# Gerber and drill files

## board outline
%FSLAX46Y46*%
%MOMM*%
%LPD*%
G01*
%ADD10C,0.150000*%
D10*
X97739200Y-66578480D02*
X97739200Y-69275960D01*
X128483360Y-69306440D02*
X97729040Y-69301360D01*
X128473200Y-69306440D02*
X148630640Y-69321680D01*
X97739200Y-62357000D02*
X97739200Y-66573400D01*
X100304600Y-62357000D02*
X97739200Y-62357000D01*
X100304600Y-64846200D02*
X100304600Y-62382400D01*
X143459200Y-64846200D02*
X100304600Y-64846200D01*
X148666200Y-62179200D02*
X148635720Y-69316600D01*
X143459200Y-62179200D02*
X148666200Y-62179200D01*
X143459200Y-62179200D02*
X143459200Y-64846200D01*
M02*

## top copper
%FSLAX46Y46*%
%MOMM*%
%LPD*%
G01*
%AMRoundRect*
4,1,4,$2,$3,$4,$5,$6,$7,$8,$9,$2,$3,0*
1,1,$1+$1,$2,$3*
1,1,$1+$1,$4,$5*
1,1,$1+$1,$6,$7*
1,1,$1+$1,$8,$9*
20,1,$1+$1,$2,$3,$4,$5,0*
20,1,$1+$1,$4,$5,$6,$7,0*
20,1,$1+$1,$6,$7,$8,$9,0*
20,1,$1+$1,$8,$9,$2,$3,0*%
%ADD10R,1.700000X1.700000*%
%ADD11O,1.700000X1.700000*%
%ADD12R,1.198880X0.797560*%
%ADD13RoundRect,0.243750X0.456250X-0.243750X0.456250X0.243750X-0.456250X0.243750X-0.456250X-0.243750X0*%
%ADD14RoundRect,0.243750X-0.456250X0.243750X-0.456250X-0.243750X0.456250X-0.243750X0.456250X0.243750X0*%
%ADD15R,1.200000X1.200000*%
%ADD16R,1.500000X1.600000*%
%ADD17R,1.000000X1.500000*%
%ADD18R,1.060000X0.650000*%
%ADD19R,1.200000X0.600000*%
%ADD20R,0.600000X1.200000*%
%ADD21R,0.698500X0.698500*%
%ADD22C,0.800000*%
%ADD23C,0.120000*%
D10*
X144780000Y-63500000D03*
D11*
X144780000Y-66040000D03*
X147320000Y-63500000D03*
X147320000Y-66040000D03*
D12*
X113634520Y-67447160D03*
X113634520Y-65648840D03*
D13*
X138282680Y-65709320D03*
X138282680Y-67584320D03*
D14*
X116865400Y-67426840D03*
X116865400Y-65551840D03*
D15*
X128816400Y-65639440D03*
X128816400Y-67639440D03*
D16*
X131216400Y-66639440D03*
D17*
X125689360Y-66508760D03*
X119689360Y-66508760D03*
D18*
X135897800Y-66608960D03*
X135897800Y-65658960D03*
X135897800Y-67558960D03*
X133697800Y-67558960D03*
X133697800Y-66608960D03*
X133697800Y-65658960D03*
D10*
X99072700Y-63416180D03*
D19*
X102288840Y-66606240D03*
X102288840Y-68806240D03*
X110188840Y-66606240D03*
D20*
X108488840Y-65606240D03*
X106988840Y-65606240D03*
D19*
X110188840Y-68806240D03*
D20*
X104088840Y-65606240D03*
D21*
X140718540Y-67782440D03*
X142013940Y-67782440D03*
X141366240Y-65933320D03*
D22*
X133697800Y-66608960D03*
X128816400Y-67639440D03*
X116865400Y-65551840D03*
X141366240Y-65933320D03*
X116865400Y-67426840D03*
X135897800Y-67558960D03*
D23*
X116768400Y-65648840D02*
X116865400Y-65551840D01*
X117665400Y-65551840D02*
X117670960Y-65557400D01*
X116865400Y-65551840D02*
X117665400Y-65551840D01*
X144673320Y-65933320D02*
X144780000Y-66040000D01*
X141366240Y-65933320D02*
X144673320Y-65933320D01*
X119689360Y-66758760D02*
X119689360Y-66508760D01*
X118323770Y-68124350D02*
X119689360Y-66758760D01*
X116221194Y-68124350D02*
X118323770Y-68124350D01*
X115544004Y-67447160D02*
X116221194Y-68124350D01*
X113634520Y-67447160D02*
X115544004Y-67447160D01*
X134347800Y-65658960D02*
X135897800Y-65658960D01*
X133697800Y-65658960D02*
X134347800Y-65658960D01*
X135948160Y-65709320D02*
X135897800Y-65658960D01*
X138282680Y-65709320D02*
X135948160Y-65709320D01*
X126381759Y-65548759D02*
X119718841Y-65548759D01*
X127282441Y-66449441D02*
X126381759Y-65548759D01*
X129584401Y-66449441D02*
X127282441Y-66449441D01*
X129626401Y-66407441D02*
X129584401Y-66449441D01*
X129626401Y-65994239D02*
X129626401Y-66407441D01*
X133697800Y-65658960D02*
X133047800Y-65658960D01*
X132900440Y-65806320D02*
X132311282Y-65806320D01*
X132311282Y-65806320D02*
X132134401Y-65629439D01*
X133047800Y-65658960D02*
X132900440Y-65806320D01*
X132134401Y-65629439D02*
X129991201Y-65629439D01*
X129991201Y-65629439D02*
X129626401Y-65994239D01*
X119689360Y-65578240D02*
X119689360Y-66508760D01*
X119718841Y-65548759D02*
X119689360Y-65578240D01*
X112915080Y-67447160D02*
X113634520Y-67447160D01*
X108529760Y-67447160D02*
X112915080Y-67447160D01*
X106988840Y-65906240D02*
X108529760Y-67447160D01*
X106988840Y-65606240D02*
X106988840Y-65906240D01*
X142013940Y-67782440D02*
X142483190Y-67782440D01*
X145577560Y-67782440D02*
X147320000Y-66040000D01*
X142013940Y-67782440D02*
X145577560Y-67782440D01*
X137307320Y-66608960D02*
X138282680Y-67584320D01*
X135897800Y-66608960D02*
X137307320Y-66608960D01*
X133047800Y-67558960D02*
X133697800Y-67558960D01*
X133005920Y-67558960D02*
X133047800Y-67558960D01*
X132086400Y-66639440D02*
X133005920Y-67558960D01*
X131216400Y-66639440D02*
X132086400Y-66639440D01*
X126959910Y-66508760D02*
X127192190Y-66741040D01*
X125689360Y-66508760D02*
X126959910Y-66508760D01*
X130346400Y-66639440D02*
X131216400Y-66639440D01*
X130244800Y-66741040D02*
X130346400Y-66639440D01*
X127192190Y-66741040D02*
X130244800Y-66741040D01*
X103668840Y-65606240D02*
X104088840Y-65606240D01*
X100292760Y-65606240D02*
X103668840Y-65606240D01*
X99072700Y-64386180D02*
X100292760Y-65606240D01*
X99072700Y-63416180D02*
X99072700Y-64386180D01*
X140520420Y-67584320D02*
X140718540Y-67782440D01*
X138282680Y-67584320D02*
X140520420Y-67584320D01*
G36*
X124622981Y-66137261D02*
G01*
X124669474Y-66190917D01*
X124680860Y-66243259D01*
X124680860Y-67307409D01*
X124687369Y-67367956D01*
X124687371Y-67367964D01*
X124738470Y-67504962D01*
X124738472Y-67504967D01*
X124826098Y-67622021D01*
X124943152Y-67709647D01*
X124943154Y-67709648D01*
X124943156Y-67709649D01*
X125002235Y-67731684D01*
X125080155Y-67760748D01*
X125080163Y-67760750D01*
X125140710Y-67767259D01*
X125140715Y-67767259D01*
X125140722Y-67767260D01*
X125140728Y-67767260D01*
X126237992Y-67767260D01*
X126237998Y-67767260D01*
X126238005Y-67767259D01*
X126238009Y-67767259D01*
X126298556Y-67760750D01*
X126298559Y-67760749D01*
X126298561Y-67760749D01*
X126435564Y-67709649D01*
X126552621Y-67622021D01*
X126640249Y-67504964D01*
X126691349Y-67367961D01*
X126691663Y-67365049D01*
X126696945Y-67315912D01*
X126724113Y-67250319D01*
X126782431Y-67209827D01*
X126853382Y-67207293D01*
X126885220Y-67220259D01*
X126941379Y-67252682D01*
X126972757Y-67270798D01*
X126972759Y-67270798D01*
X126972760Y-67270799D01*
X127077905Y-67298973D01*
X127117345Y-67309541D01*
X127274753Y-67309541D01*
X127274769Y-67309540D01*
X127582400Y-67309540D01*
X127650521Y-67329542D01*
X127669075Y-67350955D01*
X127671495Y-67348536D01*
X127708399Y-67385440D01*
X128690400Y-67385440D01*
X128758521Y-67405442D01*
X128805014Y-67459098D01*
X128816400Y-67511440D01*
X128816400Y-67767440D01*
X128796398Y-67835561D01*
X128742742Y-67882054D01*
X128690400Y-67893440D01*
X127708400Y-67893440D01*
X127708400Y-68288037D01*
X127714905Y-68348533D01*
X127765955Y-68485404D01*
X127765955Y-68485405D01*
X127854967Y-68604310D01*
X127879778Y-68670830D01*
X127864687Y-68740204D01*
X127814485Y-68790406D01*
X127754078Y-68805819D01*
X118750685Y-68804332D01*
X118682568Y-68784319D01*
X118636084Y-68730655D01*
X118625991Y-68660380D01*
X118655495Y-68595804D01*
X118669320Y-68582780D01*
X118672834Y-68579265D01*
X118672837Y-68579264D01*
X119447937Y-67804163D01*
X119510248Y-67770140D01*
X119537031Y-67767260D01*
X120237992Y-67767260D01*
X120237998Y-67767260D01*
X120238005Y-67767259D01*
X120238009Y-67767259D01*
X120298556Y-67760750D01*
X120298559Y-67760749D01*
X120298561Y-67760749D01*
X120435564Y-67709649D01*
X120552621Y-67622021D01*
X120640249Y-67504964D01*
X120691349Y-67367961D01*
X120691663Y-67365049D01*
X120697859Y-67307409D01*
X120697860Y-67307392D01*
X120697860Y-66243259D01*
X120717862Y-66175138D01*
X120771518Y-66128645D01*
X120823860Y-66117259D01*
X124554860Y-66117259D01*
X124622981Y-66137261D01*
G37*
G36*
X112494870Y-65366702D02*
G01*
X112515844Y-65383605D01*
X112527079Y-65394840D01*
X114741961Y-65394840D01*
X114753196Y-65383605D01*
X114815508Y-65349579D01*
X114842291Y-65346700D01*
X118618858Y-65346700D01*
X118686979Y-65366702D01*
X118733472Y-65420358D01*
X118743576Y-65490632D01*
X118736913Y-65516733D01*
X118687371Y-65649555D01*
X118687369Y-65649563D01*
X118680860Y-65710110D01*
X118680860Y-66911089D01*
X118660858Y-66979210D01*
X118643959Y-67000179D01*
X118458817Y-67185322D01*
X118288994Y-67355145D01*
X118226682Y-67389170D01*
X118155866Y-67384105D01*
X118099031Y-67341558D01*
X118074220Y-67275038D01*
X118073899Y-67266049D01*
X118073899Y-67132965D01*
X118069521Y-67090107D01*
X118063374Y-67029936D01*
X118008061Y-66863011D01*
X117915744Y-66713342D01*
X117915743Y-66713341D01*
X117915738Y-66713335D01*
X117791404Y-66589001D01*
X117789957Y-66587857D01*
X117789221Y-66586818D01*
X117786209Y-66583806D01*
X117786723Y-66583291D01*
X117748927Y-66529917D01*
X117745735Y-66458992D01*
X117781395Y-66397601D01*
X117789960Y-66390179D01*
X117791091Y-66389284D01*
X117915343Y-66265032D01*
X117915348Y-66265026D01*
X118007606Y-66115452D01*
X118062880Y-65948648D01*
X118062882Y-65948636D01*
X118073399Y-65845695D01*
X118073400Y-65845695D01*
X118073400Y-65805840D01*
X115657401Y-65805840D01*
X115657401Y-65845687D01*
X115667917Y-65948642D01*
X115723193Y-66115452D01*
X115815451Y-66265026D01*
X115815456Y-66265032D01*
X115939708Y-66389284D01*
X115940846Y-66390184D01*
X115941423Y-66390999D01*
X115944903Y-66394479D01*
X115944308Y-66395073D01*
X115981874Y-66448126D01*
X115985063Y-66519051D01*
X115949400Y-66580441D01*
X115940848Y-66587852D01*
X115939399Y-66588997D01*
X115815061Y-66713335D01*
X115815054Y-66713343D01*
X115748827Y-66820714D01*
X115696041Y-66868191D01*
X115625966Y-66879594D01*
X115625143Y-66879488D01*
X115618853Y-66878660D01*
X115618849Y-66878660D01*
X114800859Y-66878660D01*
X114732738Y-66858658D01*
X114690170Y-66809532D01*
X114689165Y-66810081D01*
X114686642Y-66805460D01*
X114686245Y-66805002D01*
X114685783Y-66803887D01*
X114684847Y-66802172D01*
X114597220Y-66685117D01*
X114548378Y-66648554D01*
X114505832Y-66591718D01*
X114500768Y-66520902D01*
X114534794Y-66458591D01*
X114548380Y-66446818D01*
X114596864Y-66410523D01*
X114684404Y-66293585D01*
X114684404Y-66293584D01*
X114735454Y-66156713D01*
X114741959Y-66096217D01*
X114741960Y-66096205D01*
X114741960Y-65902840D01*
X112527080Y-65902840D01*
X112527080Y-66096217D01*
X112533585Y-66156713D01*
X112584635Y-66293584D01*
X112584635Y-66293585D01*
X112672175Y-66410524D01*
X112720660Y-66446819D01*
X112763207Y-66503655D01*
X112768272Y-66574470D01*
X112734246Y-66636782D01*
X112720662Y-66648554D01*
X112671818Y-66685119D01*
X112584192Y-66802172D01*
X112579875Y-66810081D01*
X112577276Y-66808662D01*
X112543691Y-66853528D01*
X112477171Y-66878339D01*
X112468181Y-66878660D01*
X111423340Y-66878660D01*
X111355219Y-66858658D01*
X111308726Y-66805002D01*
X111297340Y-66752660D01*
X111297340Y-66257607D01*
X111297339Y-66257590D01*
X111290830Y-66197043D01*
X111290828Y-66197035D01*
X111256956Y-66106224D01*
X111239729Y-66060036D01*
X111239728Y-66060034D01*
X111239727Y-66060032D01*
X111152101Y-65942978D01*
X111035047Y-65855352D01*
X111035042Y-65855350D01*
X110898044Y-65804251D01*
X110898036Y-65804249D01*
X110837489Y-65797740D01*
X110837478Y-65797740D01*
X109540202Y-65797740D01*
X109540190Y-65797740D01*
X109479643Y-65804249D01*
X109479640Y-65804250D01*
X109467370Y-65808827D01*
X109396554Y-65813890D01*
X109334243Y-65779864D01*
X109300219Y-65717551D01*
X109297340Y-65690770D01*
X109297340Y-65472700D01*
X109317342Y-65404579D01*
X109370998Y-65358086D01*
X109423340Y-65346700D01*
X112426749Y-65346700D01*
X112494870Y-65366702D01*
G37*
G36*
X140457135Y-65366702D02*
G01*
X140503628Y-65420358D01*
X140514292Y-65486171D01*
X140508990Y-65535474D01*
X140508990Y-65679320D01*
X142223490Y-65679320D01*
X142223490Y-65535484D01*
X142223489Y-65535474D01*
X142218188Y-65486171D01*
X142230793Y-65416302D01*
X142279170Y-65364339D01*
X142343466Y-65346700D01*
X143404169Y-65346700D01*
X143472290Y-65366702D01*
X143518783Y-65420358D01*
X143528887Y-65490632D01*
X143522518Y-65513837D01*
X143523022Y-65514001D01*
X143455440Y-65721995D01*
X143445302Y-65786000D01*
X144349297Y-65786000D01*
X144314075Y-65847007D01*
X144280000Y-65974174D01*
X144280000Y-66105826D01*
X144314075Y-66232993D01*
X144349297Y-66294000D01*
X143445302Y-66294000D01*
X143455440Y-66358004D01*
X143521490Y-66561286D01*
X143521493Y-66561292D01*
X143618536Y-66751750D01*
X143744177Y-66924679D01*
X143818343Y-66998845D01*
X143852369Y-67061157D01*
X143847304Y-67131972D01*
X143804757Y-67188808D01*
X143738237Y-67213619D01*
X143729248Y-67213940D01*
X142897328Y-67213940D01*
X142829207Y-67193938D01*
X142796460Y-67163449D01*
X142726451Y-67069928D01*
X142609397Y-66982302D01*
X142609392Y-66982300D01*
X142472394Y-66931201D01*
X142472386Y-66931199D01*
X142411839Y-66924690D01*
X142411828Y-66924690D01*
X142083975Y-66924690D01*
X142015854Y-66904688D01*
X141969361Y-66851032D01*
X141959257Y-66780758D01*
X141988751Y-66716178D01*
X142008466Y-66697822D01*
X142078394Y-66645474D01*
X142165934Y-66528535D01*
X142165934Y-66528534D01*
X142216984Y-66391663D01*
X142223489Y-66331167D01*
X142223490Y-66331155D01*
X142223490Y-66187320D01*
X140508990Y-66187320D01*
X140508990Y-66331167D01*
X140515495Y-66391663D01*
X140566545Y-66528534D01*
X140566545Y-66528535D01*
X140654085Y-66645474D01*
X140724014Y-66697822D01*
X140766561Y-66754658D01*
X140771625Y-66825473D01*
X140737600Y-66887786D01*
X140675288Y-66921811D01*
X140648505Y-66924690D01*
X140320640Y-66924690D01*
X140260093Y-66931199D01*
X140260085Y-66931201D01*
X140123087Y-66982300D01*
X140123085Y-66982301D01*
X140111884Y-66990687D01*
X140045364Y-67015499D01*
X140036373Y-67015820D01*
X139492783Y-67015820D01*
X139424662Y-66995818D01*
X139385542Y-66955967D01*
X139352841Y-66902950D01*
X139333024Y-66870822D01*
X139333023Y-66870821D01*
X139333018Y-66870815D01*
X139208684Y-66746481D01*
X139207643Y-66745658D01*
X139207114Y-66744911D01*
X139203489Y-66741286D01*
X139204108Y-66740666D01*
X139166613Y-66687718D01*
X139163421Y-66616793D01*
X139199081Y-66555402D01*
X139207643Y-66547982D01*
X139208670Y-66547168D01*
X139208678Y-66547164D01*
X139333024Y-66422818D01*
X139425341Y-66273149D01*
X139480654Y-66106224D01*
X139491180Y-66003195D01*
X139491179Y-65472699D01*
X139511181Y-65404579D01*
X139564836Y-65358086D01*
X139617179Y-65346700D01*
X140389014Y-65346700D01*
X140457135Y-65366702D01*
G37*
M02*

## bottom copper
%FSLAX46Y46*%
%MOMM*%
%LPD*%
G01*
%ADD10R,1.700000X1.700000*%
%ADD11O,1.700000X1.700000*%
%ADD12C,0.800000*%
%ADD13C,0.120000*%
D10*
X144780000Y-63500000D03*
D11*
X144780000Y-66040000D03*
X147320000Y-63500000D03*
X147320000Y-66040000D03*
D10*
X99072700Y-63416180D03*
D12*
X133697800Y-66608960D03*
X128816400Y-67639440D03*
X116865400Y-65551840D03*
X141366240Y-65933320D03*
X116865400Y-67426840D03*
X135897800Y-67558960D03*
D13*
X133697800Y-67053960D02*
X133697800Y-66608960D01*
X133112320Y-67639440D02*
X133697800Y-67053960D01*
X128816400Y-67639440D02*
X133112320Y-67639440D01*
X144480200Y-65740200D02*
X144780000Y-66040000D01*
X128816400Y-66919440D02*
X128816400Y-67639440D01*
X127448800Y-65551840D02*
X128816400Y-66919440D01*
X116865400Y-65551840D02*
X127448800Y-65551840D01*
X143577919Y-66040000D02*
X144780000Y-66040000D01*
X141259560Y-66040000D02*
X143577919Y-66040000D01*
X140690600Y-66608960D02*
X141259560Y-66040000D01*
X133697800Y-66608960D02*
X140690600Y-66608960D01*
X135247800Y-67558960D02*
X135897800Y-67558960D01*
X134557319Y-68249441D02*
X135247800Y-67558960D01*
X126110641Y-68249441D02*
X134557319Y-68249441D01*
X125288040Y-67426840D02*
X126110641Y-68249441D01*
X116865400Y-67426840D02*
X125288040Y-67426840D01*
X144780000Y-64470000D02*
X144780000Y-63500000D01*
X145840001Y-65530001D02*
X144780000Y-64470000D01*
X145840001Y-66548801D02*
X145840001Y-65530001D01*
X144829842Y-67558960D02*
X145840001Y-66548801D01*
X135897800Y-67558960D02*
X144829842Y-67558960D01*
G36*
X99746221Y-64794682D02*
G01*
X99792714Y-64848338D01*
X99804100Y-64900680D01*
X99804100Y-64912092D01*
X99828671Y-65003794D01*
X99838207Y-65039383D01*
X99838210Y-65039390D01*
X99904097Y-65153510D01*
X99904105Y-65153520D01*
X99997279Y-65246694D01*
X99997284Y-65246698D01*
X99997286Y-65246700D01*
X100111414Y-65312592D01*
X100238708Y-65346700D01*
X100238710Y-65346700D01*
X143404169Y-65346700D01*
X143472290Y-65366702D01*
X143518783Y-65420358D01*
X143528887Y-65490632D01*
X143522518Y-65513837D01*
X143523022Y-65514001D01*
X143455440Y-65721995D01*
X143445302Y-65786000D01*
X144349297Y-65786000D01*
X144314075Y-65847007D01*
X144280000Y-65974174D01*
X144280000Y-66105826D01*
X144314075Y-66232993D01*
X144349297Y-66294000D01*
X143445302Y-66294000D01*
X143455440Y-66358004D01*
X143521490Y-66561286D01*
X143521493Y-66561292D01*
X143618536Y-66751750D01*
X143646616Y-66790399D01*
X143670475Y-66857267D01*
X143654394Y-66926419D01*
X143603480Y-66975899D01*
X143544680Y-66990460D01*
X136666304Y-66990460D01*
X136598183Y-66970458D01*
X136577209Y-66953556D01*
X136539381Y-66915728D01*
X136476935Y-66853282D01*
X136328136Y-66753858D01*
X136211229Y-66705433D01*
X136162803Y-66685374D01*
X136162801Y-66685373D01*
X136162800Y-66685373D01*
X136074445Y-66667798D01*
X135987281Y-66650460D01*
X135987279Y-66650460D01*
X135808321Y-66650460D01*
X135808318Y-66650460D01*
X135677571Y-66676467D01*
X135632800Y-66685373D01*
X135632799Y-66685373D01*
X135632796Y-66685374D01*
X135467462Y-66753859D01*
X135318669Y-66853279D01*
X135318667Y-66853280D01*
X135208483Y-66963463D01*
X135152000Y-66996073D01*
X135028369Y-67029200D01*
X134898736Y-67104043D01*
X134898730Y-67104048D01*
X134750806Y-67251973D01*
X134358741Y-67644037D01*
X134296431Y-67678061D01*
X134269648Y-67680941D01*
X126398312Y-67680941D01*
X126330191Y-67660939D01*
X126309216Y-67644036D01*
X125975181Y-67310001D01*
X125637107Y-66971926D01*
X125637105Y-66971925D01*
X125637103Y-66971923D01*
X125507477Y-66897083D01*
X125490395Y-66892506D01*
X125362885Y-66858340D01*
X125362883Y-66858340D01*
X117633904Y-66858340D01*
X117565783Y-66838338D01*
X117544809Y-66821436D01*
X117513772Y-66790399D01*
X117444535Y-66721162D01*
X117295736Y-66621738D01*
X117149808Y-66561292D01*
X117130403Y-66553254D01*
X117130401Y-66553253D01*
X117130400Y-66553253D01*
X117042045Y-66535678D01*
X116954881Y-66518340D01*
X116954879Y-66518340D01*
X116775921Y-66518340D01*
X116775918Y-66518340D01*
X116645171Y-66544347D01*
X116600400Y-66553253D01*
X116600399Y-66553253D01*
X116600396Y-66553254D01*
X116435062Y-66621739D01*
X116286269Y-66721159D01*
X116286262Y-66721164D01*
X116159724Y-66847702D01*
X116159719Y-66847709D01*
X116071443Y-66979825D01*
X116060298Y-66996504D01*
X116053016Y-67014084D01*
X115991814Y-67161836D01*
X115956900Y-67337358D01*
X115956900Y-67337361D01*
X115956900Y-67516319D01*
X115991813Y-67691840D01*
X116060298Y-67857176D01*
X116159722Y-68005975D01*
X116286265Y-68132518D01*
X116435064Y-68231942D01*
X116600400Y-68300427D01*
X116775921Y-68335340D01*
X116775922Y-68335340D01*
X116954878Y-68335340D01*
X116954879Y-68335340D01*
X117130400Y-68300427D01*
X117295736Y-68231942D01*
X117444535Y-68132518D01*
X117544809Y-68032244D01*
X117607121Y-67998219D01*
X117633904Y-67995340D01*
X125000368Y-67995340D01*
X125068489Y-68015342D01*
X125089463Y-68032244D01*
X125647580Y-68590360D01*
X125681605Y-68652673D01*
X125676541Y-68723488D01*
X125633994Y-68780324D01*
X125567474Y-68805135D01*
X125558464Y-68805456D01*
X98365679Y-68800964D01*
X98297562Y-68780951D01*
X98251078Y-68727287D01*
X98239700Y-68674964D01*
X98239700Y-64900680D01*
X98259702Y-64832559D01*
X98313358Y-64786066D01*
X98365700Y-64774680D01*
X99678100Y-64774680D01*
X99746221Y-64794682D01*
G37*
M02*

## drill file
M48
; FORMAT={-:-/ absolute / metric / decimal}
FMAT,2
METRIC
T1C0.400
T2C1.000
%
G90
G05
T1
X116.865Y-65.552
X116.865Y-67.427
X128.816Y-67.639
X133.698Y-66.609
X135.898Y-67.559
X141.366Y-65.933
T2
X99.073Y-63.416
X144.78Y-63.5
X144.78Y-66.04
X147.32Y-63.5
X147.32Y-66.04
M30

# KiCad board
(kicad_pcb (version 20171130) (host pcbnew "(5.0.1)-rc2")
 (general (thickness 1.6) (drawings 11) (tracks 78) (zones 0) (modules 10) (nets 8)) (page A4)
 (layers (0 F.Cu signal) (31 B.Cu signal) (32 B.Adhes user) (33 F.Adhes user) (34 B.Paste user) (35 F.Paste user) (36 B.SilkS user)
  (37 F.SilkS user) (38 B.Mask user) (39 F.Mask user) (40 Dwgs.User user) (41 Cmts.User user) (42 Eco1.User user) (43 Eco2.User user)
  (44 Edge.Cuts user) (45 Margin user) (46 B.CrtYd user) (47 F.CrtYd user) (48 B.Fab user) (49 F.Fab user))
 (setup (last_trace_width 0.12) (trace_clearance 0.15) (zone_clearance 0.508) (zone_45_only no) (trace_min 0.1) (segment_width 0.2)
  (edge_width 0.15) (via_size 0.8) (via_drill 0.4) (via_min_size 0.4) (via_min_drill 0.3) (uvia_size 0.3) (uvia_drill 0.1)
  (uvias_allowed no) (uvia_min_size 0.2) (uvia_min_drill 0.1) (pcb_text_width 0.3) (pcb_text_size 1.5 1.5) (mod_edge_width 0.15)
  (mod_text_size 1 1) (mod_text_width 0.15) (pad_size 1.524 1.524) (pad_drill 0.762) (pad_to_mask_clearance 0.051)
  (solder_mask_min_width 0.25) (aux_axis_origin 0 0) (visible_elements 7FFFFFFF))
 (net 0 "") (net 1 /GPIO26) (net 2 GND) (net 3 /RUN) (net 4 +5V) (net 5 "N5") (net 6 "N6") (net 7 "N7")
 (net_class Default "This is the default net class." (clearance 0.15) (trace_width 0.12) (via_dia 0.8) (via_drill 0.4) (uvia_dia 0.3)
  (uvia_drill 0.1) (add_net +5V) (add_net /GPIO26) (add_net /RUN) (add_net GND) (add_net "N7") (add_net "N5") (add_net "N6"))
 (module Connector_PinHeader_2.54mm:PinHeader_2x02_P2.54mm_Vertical (layer B.Cu) (at 144.78 63.5 270)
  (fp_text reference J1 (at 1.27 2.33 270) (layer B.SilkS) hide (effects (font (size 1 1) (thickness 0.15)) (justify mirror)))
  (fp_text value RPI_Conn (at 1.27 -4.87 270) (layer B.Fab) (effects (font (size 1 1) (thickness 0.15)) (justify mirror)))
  (pad 1 thru_hole rect (at 0 0 270) (size 1.7 1.7) (drill 1) (layers *.Cu *.Mask) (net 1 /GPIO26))
  (pad 2 thru_hole oval (at 2.54 0 270) (size 1.7 1.7) (drill 1) (layers *.Cu *.Mask) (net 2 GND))
  (pad 3 thru_hole oval (at 0 -2.54 270) (size 1.7 1.7) (drill 1) (layers *.Cu *.Mask) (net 2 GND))
  (pad 4 thru_hole oval (at 2.54 -2.54 270) (size 1.7 1.7) (drill 1) (layers *.Cu *.Mask) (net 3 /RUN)))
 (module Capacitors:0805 (layer F.Cu) (at 113.63452 66.548 270)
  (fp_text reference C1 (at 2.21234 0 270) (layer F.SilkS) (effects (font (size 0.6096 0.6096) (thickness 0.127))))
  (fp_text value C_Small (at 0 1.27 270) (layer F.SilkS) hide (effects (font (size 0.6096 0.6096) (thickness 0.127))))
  (pad 2 smd rect (at 0.89916 0 270) (size 0.79756 1.19888) (layers F.Cu F.Paste F.Mask) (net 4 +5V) (solder_mask_margin 0.1016))
  (pad 1 smd rect (at -0.89916 0 270) (size 0.79756 1.19888) (layers F.Cu F.Paste F.Mask) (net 2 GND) (solder_mask_margin 0.1016)))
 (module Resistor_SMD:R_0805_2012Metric (layer F.Cu) (at 138.28268 66.64682 90)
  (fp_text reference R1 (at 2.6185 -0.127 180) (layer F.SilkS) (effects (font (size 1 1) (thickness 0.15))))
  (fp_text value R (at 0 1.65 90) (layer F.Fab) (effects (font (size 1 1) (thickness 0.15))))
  (pad 2 smd roundrect (at 0.9375 0 90) (size 0.975 1.4) (layers F.Cu F.Paste F.Mask) (roundrect_rratio 0.25) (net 4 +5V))
  (pad 1 smd roundrect (at -0.9375 0 90) (size 0.975 1.4) (layers F.Cu F.Paste F.Mask) (roundrect_rratio 0.25) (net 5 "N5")))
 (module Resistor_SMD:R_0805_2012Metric (layer F.Cu) (at 116.8654 66.48934 270)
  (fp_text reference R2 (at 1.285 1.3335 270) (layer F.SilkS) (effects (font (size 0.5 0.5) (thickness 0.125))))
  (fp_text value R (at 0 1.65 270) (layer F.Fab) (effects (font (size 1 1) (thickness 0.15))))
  (pad 2 smd roundrect (at 0.9375 0 270) (size 0.975 1.4) (layers F.Cu F.Paste F.Mask) (roundrect_rratio 0.25) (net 1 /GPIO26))
  (pad 1 smd roundrect (at -0.9375 0 270) (size 0.975 1.4) (layers F.Cu F.Paste F.Mask) (roundrect_rratio 0.25) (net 2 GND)))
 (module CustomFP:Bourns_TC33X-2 (layer F.Cu) (at 131.2164 66.63944 270)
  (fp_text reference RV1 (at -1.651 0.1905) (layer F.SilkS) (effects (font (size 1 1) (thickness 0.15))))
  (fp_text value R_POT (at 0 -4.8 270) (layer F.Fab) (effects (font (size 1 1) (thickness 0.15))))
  (pad 3 smd rect (at -1 2.4 270) (size 1.2 1.2) (layers F.Cu F.Paste F.Mask))
  (pad 2 smd rect (at 1 2.4 270) (size 1.2 1.2) (layers F.Cu F.Paste F.Mask) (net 2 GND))
  (pad 1 smd rect (at 0 0 270) (size 1.6 1.5) (layers F.Cu F.Paste F.Mask) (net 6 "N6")))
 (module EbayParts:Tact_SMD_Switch (layer F.Cu) (at 125.68936 65.00876 180)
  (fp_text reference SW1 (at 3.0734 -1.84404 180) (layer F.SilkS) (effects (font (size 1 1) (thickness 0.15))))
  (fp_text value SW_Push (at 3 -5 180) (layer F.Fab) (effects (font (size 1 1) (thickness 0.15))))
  (pad 1 smd rect (at 0 -1.5 180) (size 1 1.5) (layers F.Cu F.Paste F.Mask) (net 6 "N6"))
  (pad 2 smd rect (at 6 -1.5 180) (size 1 1.5) (layers F.Cu F.Paste F.Mask) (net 4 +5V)))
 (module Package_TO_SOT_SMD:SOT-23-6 (layer F.Cu) (at 134.7978 66.60896)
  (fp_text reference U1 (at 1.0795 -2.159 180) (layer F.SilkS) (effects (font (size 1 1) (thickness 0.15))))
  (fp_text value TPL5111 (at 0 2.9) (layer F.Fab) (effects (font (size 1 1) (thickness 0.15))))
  (pad 5 smd rect (at 1.1 0) (size 1.06 0.65) (layers F.Cu F.Paste F.Mask) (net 5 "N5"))
  (pad 6 smd rect (at 1.1 -0.95) (size 1.06 0.65) (layers F.Cu F.Paste F.Mask) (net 4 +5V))
  (pad 4 smd rect (at 1.1 0.95) (size 1.06 0.65) (layers F.Cu F.Paste F.Mask) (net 1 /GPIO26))
  (pad 3 smd rect (at -1.1 0.95) (size 1.06 0.65) (layers F.Cu F.Paste F.Mask) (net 6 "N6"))
  (pad 2 smd rect (at -1.1 0) (size 1.06 0.65) (layers F.Cu F.Paste F.Mask) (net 2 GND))
  (pad 1 smd rect (at -1.1 -0.95) (size 1.06 0.65) (layers F.Cu F.Paste F.Mask) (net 4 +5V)))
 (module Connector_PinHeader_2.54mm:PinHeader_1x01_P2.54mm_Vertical (layer F.Cu) (at 99.0727 63.41618)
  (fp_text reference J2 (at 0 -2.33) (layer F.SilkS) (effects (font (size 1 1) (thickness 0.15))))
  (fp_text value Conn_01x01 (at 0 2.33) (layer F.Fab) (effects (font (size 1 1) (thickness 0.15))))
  (pad 1 thru_hole rect (at 0 0) (size 1.7 1.7) (drill 1) (layers *.Cu *.Mask) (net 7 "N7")))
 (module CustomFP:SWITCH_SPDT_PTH (layer F.Cu) (at 106.28884 67.70624 90)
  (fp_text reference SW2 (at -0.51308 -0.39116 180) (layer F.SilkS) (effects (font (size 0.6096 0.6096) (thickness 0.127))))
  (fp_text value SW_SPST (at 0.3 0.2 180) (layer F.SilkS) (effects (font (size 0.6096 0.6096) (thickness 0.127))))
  (pad "" smd rect (at 1.1 -4 180) (size 1.2 0.6) (layers F.Cu F.Paste F.Mask) (solder_mask_margin 0.1016))
  (pad "" smd rect (at -1.1 -4 180) (size 1.2 0.6) (layers F.Cu F.Paste F.Mask) (solder_mask_margin 0.1016))
  (pad "" smd rect (at 1.1 3.9 180) (size 1.2 0.6) (layers F.Cu F.Paste F.Mask) (solder_mask_margin 0.1016))
  (pad 3 smd rect (at 2.1 2.2 90) (size 1.2 0.6) (layers F.Cu F.Paste F.Mask) (solder_mask_margin 0.1016))
  (pad 2 smd rect (at 2.1 0.7 90) (size 1.2 0.6) (layers F.Cu F.Paste F.Mask) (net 4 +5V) (solder_mask_margin 0.1016))
  (pad "" smd rect (at -1.1 3.9 180) (size 1.2 0.6) (layers F.Cu F.Paste F.Mask) (solder_mask_margin 0.1016))
  (pad 1 smd rect (at 2.1 -2.2 90) (size 1.2 0.6) (layers F.Cu F.Paste F.Mask) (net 7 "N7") (solder_mask_margin 0.1016)))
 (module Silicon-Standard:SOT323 (layer F.Cu) (at 141.36624 66.85788)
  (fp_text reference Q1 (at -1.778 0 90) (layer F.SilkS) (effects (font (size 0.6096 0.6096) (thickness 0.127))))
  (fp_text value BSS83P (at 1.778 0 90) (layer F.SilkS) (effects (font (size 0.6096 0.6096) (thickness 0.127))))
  (pad 1 smd rect (at -0.6477 0.92456) (size 0.6985 0.6985) (layers F.Cu F.Paste F.Mask) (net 5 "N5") (solder_mask_margin 0.1016))
  (pad 2 smd rect (at 0.6477 0.92456) (size 0.6985 0.6985) (layers F.Cu F.Paste F.Mask) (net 3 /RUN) (solder_mask_margin 0.1016))
  (pad 3 smd rect (at 0 -0.92456) (size 0.6985 0.6985) (layers F.Cu F.Paste F.Mask) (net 2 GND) (solder_mask_margin 0.1016)))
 (gr_line (start 97.7392 66.57848) (end 97.7392 69.27596) (layer Edge.Cuts) (width 0.15))
 (gr_line (start 128.48336 69.30644) (end 97.72904 69.30136) (layer Edge.Cuts) (width 0.15))
 (gr_line (start 128.4732 69.30644) (end 148.63064 69.32168) (layer Edge.Cuts) (width 0.15))
 (gr_line (start 97.7392 62.357) (end 97.7392 66.5734) (layer Edge.Cuts) (width 0.15))
 (gr_line (start 100.3046 62.357) (end 97.7392 62.357) (layer Edge.Cuts) (width 0.15))
 (gr_line (start 100.3046 64.8462) (end 100.3046 62.3824) (layer Edge.Cuts) (width 0.15))
 (gr_line (start 143.4592 64.8462) (end 100.3046 64.8462) (layer Edge.Cuts) (width 0.15))
 (gr_line (start 148.6662 62.1792) (end 148.63572 69.3166) (layer Edge.Cuts) (width 0.15))
 (gr_line (start 143.4592 62.1792) (end 148.6662 62.1792) (layer Edge.Cuts) (width 0.15))
 (gr_line (start 143.4592 62.1792) (end 143.4592 64.8462) (layer Edge.Cuts) (width 0.15))
 (segment (start 116.7684 65.64884) (end 116.8654 65.55184) (width 0.12) (layer F.Cu) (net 2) (status 30))
 (segment (start 117.6654 65.55184) (end 117.67096 65.5574) (width 0.12) (layer F.Cu) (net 2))
 (segment (start 116.8654 65.55184) (end 117.6654 65.55184) (width 0.12) (layer F.Cu) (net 2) (status 10))
 (via (at 133.6978 66.60896) (size 0.8) (drill 0.4) (layers F.Cu B.Cu) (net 2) (status 30))
 (via (at 128.8164 67.63944) (size 0.8) (drill 0.4) (layers F.Cu B.Cu) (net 2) (status 30))
 (via (at 116.8654 65.55184) (size 0.8) (drill 0.4) (layers F.Cu B.Cu) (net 2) (status 30))
 (segment (start 133.6978 67.05396) (end 133.6978 66.60896) (width 0.12) (layer B.Cu) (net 2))
 (segment (start 133.11232 67.63944) (end 133.6978 67.05396) (width 0.12) (layer B.Cu) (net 2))
 (segment (start 128.8164 67.63944) (end 133.11232 67.63944) (width 0.12) (layer B.Cu) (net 2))
 (segment (start 144.4802 65.7402) (end 144.78 66.04) (width 0.12) (layer B.Cu) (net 2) (status 30))
 (segment (start 128.8164 66.91944) (end 128.8164 67.63944) (width 0.12) (layer B.Cu) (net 2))
 (segment (start 127.4488 65.55184) (end 128.8164 66.91944) (width 0.12) (layer B.Cu) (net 2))
 (segment (start 116.8654 65.55184) (end 127.4488 65.55184) (width 0.12) (layer B.Cu) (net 2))
 (segment (start 144.67332 65.93332) (end 144.78 66.04) (width 0.12) (layer F.Cu) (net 2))
 (segment (start 141.36624 65.93332) (end 144.67332 65.93332) (width 0.12) (layer F.Cu) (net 2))
 (via (at 141.36624 65.93332) (size 0.8) (drill 0.4) (layers F.Cu B.Cu) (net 2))
 (segment (start 143.577919 66.04) (end 144.78 66.04) (width 0.12) (layer B.Cu) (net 2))
 (segment (start 141.25956 66.04) (end 143.577919 66.04) (width 0.12) (layer B.Cu) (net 2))
 (segment (start 140.6906 66.60896) (end 141.25956 66.04) (width 0.12) (layer B.Cu) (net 2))
 (segment (start 133.6978 66.60896) (end 140.6906 66.60896) (width 0.12) (layer B.Cu) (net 2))
 (segment (start 119.68936 66.75876) (end 119.68936 66.50876) (width 0.12) (layer F.Cu) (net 4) (status 30))
 (segment (start 118.32377 68.12435) (end 119.68936 66.75876) (width 0.12) (layer F.Cu) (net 4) (status 20))
 (segment (start 116.221194 68.12435) (end 118.32377 68.12435) (width 0.12) (layer F.Cu) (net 4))
 (segment (start 115.544004 67.44716) (end 116.221194 68.12435) (width 0.12) (layer F.Cu) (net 4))
 (segment (start 113.63452 67.44716) (end 115.544004 67.44716) (width 0.12) (layer F.Cu) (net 4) (status 10))
 (segment (start 134.3478 65.65896) (end 135.8978 65.65896) (width 0.12) (layer F.Cu) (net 4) (status 20))
 (segment (start 133.6978 65.65896) (end 134.3478 65.65896) (width 0.12) (layer F.Cu) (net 4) (status 10))
 (segment (start 135.94816 65.70932) (end 135.8978 65.65896) (width 0.12) (layer F.Cu) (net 4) (status 30))
 (segment (start 138.28268 65.70932) (end 135.94816 65.70932) (width 0.12) (layer F.Cu) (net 4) (status 30))
 (segment (start 126.381759 65.548759) (end 119.718841 65.548759) (width 0.12) (layer F.Cu) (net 4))
 (segment (start 127.282441 66.449441) (end 126.381759 65.548759) (width 0.12) (layer F.Cu) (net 4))
 (segment (start 129.584401 66.449441) (end 127.282441 66.449441) (width 0.12) (layer F.Cu) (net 4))
 (segment (start 129.626401 66.407441) (end 129.584401 66.449441) (width 0.12) (layer F.Cu) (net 4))
 (segment (start 129.626401 65.994239) (end 129.626401 66.407441) (width 0.12) (layer F.Cu) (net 4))
 (segment (start 133.6978 65.65896) (end 133.0478 65.65896) (width 0.12) (layer F.Cu) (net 4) (status 10))
 (segment (start 132.90044 65.80632) (end 132.311282 65.80632) (width 0.12) (layer F.Cu) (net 4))
 (segment (start 132.311282 65.80632) (end 132.134401 65.629439) (width 0.12) (layer F.Cu) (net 4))
 (segment (start 133.0478 65.65896) (end 132.90044 65.80632) (width 0.12) (layer F.Cu) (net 4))
 (segment (start 132.134401 65.629439) (end 129.991201 65.629439) (width 0.12) (layer F.Cu) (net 4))
 (segment (start 129.991201 65.629439) (end 129.626401 65.994239) (width 0.12) (layer F.Cu) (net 4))
 (segment (start 119.68936 65.57824) (end 119.68936 66.50876) (width 0.12) (layer F.Cu) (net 4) (status 20))
 (segment (start 119.718841 65.548759) (end 119.68936 65.57824) (width 0.12) (layer F.Cu) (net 4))
 (segment (start 112.91508 67.44716) (end 113.63452 67.44716) (width 0.12) (layer F.Cu) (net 4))
 (segment (start 108.52976 67.44716) (end 112.91508 67.44716) (width 0.12) (layer F.Cu) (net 4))
 (segment (start 106.98884 65.90624) (end 108.52976 67.44716) (width 0.12) (layer F.Cu) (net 4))
 (segment (start 106.98884 65.60624) (end 106.98884 65.90624) (width 0.12) (layer F.Cu) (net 4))
 (via (at 116.8654 67.42684) (size 0.8) (drill 0.4) (layers F.Cu B.Cu) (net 1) (status 30))
 (via (at 135.8978 67.55896) (size 0.8) (drill 0.4) (layers F.Cu B.Cu) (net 1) (status 30))
 (segment (start 135.2478 67.55896) (end 135.8978 67.55896) (width 0.12) (layer B.Cu) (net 1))
 (segment (start 134.557319 68.249441) (end 135.2478 67.55896) (width 0.12) (layer B.Cu) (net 1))
 (segment (start 126.110641 68.249441) (end 134.557319 68.249441) (width 0.12) (layer B.Cu) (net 1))
 (segment (start 125.28804 67.42684) (end 126.110641 68.249441) (width 0.12) (layer B.Cu) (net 1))
 (segment (start 116.8654 67.42684) (end 125.28804 67.42684) (width 0.12) (layer B.Cu) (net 1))
 (segment (start 144.78 64.47) (end 144.78 63.5) (width 0.12) (layer B.Cu) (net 1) (status 20))
 (segment (start 145.840001 65.530001) (end 144.78 64.47) (width 0.12) (layer B.Cu) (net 1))
 (segment (start 145.840001 66.548801) (end 145.840001 65.530001) (width 0.12) (layer B.Cu) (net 1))
 (segment (start 144.829842 67.55896) (end 145.840001 66.548801) (width 0.12) (layer B.Cu) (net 1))
 (segment (start 135.8978 67.55896) (end 144.829842 67.55896) (width 0.12) (layer B.Cu) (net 1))
 (segment (start 142.01394 67.78244) (end 142.48319 67.78244) (width 0.12) (layer F.Cu) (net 3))
 (segment (start 145.57756 67.78244) (end 147.32 66.04) (width 0.12) (layer F.Cu) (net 3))
 (segment (start 142.01394 67.78244) (end 145.57756 67.78244) (width 0.12) (layer F.Cu) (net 3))
 (segment (start 137.30732 66.60896) (end 138.28268 67.58432) (width 0.12) (layer F.Cu) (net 5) (status 20))
 (segment (start 135.8978 66.60896) (end 137.30732 66.60896) (width 0.12) (layer F.Cu) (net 5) (status 10))
 (segment (start 133.0478 67.55896) (end 133.6978 67.55896) (width 0.12) (layer F.Cu) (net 6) (status 20))
 (segment (start 133.00592 67.55896) (end 133.0478 67.55896) (width 0.12) (layer F.Cu) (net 6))
 (segment (start 132.0864 66.63944) (end 133.00592 67.55896) (width 0.12) (layer F.Cu) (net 6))
 (segment (start 131.2164 66.63944) (end 132.0864 66.63944) (width 0.12) (layer F.Cu) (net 6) (status 10))
 (segment (start 126.95991 66.50876) (end 127.19219 66.74104) (width 0.12) (layer F.Cu) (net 6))
 (segment (start 125.68936 66.50876) (end 126.95991 66.50876) (width 0.12) (layer F.Cu) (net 6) (status 10))
 (segment (start 130.3464 66.63944) (end 131.2164 66.63944) (width 0.12) (layer F.Cu) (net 6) (status 20))
 (segment (start 130.2448 66.74104) (end 130.3464 66.63944) (width 0.12) (layer F.Cu) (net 6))
 (segment (start 127.19219 66.74104) (end 130.2448 66.74104) (width 0.12) (layer F.Cu) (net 6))
 (segment (start 103.66884 65.60624) (end 104.08884 65.60624) (width 0.12) (layer F.Cu) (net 7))
 (segment (start 100.29276 65.60624) (end 103.66884 65.60624) (width 0.12) (layer F.Cu) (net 7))
 (segment (start 99.0727 64.38618) (end 100.29276 65.60624) (width 0.12) (layer F.Cu) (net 7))
 (segment (start 99.0727 63.41618) (end 99.0727 64.38618) (width 0.12) (layer F.Cu) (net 7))
 (segment (start 140.52042 67.58432) (end 140.71854 67.78244) (width 0.12) (layer F.Cu) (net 5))
 (segment (start 138.28268 67.58432) (end 140.52042 67.58432) (width 0.12) (layer F.Cu) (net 5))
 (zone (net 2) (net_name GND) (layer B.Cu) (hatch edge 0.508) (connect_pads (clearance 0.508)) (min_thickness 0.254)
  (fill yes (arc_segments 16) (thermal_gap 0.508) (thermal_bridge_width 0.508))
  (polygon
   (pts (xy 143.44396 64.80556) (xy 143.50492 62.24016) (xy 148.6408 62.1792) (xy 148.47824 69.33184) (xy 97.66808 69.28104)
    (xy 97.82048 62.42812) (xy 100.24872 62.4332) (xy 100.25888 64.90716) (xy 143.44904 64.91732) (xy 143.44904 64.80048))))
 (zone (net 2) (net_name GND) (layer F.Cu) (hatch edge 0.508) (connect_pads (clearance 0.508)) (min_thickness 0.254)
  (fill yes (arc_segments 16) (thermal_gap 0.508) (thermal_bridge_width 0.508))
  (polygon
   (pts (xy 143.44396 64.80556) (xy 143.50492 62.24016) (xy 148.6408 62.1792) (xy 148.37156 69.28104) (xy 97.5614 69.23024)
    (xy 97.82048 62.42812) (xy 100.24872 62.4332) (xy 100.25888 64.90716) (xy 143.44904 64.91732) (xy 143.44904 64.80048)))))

